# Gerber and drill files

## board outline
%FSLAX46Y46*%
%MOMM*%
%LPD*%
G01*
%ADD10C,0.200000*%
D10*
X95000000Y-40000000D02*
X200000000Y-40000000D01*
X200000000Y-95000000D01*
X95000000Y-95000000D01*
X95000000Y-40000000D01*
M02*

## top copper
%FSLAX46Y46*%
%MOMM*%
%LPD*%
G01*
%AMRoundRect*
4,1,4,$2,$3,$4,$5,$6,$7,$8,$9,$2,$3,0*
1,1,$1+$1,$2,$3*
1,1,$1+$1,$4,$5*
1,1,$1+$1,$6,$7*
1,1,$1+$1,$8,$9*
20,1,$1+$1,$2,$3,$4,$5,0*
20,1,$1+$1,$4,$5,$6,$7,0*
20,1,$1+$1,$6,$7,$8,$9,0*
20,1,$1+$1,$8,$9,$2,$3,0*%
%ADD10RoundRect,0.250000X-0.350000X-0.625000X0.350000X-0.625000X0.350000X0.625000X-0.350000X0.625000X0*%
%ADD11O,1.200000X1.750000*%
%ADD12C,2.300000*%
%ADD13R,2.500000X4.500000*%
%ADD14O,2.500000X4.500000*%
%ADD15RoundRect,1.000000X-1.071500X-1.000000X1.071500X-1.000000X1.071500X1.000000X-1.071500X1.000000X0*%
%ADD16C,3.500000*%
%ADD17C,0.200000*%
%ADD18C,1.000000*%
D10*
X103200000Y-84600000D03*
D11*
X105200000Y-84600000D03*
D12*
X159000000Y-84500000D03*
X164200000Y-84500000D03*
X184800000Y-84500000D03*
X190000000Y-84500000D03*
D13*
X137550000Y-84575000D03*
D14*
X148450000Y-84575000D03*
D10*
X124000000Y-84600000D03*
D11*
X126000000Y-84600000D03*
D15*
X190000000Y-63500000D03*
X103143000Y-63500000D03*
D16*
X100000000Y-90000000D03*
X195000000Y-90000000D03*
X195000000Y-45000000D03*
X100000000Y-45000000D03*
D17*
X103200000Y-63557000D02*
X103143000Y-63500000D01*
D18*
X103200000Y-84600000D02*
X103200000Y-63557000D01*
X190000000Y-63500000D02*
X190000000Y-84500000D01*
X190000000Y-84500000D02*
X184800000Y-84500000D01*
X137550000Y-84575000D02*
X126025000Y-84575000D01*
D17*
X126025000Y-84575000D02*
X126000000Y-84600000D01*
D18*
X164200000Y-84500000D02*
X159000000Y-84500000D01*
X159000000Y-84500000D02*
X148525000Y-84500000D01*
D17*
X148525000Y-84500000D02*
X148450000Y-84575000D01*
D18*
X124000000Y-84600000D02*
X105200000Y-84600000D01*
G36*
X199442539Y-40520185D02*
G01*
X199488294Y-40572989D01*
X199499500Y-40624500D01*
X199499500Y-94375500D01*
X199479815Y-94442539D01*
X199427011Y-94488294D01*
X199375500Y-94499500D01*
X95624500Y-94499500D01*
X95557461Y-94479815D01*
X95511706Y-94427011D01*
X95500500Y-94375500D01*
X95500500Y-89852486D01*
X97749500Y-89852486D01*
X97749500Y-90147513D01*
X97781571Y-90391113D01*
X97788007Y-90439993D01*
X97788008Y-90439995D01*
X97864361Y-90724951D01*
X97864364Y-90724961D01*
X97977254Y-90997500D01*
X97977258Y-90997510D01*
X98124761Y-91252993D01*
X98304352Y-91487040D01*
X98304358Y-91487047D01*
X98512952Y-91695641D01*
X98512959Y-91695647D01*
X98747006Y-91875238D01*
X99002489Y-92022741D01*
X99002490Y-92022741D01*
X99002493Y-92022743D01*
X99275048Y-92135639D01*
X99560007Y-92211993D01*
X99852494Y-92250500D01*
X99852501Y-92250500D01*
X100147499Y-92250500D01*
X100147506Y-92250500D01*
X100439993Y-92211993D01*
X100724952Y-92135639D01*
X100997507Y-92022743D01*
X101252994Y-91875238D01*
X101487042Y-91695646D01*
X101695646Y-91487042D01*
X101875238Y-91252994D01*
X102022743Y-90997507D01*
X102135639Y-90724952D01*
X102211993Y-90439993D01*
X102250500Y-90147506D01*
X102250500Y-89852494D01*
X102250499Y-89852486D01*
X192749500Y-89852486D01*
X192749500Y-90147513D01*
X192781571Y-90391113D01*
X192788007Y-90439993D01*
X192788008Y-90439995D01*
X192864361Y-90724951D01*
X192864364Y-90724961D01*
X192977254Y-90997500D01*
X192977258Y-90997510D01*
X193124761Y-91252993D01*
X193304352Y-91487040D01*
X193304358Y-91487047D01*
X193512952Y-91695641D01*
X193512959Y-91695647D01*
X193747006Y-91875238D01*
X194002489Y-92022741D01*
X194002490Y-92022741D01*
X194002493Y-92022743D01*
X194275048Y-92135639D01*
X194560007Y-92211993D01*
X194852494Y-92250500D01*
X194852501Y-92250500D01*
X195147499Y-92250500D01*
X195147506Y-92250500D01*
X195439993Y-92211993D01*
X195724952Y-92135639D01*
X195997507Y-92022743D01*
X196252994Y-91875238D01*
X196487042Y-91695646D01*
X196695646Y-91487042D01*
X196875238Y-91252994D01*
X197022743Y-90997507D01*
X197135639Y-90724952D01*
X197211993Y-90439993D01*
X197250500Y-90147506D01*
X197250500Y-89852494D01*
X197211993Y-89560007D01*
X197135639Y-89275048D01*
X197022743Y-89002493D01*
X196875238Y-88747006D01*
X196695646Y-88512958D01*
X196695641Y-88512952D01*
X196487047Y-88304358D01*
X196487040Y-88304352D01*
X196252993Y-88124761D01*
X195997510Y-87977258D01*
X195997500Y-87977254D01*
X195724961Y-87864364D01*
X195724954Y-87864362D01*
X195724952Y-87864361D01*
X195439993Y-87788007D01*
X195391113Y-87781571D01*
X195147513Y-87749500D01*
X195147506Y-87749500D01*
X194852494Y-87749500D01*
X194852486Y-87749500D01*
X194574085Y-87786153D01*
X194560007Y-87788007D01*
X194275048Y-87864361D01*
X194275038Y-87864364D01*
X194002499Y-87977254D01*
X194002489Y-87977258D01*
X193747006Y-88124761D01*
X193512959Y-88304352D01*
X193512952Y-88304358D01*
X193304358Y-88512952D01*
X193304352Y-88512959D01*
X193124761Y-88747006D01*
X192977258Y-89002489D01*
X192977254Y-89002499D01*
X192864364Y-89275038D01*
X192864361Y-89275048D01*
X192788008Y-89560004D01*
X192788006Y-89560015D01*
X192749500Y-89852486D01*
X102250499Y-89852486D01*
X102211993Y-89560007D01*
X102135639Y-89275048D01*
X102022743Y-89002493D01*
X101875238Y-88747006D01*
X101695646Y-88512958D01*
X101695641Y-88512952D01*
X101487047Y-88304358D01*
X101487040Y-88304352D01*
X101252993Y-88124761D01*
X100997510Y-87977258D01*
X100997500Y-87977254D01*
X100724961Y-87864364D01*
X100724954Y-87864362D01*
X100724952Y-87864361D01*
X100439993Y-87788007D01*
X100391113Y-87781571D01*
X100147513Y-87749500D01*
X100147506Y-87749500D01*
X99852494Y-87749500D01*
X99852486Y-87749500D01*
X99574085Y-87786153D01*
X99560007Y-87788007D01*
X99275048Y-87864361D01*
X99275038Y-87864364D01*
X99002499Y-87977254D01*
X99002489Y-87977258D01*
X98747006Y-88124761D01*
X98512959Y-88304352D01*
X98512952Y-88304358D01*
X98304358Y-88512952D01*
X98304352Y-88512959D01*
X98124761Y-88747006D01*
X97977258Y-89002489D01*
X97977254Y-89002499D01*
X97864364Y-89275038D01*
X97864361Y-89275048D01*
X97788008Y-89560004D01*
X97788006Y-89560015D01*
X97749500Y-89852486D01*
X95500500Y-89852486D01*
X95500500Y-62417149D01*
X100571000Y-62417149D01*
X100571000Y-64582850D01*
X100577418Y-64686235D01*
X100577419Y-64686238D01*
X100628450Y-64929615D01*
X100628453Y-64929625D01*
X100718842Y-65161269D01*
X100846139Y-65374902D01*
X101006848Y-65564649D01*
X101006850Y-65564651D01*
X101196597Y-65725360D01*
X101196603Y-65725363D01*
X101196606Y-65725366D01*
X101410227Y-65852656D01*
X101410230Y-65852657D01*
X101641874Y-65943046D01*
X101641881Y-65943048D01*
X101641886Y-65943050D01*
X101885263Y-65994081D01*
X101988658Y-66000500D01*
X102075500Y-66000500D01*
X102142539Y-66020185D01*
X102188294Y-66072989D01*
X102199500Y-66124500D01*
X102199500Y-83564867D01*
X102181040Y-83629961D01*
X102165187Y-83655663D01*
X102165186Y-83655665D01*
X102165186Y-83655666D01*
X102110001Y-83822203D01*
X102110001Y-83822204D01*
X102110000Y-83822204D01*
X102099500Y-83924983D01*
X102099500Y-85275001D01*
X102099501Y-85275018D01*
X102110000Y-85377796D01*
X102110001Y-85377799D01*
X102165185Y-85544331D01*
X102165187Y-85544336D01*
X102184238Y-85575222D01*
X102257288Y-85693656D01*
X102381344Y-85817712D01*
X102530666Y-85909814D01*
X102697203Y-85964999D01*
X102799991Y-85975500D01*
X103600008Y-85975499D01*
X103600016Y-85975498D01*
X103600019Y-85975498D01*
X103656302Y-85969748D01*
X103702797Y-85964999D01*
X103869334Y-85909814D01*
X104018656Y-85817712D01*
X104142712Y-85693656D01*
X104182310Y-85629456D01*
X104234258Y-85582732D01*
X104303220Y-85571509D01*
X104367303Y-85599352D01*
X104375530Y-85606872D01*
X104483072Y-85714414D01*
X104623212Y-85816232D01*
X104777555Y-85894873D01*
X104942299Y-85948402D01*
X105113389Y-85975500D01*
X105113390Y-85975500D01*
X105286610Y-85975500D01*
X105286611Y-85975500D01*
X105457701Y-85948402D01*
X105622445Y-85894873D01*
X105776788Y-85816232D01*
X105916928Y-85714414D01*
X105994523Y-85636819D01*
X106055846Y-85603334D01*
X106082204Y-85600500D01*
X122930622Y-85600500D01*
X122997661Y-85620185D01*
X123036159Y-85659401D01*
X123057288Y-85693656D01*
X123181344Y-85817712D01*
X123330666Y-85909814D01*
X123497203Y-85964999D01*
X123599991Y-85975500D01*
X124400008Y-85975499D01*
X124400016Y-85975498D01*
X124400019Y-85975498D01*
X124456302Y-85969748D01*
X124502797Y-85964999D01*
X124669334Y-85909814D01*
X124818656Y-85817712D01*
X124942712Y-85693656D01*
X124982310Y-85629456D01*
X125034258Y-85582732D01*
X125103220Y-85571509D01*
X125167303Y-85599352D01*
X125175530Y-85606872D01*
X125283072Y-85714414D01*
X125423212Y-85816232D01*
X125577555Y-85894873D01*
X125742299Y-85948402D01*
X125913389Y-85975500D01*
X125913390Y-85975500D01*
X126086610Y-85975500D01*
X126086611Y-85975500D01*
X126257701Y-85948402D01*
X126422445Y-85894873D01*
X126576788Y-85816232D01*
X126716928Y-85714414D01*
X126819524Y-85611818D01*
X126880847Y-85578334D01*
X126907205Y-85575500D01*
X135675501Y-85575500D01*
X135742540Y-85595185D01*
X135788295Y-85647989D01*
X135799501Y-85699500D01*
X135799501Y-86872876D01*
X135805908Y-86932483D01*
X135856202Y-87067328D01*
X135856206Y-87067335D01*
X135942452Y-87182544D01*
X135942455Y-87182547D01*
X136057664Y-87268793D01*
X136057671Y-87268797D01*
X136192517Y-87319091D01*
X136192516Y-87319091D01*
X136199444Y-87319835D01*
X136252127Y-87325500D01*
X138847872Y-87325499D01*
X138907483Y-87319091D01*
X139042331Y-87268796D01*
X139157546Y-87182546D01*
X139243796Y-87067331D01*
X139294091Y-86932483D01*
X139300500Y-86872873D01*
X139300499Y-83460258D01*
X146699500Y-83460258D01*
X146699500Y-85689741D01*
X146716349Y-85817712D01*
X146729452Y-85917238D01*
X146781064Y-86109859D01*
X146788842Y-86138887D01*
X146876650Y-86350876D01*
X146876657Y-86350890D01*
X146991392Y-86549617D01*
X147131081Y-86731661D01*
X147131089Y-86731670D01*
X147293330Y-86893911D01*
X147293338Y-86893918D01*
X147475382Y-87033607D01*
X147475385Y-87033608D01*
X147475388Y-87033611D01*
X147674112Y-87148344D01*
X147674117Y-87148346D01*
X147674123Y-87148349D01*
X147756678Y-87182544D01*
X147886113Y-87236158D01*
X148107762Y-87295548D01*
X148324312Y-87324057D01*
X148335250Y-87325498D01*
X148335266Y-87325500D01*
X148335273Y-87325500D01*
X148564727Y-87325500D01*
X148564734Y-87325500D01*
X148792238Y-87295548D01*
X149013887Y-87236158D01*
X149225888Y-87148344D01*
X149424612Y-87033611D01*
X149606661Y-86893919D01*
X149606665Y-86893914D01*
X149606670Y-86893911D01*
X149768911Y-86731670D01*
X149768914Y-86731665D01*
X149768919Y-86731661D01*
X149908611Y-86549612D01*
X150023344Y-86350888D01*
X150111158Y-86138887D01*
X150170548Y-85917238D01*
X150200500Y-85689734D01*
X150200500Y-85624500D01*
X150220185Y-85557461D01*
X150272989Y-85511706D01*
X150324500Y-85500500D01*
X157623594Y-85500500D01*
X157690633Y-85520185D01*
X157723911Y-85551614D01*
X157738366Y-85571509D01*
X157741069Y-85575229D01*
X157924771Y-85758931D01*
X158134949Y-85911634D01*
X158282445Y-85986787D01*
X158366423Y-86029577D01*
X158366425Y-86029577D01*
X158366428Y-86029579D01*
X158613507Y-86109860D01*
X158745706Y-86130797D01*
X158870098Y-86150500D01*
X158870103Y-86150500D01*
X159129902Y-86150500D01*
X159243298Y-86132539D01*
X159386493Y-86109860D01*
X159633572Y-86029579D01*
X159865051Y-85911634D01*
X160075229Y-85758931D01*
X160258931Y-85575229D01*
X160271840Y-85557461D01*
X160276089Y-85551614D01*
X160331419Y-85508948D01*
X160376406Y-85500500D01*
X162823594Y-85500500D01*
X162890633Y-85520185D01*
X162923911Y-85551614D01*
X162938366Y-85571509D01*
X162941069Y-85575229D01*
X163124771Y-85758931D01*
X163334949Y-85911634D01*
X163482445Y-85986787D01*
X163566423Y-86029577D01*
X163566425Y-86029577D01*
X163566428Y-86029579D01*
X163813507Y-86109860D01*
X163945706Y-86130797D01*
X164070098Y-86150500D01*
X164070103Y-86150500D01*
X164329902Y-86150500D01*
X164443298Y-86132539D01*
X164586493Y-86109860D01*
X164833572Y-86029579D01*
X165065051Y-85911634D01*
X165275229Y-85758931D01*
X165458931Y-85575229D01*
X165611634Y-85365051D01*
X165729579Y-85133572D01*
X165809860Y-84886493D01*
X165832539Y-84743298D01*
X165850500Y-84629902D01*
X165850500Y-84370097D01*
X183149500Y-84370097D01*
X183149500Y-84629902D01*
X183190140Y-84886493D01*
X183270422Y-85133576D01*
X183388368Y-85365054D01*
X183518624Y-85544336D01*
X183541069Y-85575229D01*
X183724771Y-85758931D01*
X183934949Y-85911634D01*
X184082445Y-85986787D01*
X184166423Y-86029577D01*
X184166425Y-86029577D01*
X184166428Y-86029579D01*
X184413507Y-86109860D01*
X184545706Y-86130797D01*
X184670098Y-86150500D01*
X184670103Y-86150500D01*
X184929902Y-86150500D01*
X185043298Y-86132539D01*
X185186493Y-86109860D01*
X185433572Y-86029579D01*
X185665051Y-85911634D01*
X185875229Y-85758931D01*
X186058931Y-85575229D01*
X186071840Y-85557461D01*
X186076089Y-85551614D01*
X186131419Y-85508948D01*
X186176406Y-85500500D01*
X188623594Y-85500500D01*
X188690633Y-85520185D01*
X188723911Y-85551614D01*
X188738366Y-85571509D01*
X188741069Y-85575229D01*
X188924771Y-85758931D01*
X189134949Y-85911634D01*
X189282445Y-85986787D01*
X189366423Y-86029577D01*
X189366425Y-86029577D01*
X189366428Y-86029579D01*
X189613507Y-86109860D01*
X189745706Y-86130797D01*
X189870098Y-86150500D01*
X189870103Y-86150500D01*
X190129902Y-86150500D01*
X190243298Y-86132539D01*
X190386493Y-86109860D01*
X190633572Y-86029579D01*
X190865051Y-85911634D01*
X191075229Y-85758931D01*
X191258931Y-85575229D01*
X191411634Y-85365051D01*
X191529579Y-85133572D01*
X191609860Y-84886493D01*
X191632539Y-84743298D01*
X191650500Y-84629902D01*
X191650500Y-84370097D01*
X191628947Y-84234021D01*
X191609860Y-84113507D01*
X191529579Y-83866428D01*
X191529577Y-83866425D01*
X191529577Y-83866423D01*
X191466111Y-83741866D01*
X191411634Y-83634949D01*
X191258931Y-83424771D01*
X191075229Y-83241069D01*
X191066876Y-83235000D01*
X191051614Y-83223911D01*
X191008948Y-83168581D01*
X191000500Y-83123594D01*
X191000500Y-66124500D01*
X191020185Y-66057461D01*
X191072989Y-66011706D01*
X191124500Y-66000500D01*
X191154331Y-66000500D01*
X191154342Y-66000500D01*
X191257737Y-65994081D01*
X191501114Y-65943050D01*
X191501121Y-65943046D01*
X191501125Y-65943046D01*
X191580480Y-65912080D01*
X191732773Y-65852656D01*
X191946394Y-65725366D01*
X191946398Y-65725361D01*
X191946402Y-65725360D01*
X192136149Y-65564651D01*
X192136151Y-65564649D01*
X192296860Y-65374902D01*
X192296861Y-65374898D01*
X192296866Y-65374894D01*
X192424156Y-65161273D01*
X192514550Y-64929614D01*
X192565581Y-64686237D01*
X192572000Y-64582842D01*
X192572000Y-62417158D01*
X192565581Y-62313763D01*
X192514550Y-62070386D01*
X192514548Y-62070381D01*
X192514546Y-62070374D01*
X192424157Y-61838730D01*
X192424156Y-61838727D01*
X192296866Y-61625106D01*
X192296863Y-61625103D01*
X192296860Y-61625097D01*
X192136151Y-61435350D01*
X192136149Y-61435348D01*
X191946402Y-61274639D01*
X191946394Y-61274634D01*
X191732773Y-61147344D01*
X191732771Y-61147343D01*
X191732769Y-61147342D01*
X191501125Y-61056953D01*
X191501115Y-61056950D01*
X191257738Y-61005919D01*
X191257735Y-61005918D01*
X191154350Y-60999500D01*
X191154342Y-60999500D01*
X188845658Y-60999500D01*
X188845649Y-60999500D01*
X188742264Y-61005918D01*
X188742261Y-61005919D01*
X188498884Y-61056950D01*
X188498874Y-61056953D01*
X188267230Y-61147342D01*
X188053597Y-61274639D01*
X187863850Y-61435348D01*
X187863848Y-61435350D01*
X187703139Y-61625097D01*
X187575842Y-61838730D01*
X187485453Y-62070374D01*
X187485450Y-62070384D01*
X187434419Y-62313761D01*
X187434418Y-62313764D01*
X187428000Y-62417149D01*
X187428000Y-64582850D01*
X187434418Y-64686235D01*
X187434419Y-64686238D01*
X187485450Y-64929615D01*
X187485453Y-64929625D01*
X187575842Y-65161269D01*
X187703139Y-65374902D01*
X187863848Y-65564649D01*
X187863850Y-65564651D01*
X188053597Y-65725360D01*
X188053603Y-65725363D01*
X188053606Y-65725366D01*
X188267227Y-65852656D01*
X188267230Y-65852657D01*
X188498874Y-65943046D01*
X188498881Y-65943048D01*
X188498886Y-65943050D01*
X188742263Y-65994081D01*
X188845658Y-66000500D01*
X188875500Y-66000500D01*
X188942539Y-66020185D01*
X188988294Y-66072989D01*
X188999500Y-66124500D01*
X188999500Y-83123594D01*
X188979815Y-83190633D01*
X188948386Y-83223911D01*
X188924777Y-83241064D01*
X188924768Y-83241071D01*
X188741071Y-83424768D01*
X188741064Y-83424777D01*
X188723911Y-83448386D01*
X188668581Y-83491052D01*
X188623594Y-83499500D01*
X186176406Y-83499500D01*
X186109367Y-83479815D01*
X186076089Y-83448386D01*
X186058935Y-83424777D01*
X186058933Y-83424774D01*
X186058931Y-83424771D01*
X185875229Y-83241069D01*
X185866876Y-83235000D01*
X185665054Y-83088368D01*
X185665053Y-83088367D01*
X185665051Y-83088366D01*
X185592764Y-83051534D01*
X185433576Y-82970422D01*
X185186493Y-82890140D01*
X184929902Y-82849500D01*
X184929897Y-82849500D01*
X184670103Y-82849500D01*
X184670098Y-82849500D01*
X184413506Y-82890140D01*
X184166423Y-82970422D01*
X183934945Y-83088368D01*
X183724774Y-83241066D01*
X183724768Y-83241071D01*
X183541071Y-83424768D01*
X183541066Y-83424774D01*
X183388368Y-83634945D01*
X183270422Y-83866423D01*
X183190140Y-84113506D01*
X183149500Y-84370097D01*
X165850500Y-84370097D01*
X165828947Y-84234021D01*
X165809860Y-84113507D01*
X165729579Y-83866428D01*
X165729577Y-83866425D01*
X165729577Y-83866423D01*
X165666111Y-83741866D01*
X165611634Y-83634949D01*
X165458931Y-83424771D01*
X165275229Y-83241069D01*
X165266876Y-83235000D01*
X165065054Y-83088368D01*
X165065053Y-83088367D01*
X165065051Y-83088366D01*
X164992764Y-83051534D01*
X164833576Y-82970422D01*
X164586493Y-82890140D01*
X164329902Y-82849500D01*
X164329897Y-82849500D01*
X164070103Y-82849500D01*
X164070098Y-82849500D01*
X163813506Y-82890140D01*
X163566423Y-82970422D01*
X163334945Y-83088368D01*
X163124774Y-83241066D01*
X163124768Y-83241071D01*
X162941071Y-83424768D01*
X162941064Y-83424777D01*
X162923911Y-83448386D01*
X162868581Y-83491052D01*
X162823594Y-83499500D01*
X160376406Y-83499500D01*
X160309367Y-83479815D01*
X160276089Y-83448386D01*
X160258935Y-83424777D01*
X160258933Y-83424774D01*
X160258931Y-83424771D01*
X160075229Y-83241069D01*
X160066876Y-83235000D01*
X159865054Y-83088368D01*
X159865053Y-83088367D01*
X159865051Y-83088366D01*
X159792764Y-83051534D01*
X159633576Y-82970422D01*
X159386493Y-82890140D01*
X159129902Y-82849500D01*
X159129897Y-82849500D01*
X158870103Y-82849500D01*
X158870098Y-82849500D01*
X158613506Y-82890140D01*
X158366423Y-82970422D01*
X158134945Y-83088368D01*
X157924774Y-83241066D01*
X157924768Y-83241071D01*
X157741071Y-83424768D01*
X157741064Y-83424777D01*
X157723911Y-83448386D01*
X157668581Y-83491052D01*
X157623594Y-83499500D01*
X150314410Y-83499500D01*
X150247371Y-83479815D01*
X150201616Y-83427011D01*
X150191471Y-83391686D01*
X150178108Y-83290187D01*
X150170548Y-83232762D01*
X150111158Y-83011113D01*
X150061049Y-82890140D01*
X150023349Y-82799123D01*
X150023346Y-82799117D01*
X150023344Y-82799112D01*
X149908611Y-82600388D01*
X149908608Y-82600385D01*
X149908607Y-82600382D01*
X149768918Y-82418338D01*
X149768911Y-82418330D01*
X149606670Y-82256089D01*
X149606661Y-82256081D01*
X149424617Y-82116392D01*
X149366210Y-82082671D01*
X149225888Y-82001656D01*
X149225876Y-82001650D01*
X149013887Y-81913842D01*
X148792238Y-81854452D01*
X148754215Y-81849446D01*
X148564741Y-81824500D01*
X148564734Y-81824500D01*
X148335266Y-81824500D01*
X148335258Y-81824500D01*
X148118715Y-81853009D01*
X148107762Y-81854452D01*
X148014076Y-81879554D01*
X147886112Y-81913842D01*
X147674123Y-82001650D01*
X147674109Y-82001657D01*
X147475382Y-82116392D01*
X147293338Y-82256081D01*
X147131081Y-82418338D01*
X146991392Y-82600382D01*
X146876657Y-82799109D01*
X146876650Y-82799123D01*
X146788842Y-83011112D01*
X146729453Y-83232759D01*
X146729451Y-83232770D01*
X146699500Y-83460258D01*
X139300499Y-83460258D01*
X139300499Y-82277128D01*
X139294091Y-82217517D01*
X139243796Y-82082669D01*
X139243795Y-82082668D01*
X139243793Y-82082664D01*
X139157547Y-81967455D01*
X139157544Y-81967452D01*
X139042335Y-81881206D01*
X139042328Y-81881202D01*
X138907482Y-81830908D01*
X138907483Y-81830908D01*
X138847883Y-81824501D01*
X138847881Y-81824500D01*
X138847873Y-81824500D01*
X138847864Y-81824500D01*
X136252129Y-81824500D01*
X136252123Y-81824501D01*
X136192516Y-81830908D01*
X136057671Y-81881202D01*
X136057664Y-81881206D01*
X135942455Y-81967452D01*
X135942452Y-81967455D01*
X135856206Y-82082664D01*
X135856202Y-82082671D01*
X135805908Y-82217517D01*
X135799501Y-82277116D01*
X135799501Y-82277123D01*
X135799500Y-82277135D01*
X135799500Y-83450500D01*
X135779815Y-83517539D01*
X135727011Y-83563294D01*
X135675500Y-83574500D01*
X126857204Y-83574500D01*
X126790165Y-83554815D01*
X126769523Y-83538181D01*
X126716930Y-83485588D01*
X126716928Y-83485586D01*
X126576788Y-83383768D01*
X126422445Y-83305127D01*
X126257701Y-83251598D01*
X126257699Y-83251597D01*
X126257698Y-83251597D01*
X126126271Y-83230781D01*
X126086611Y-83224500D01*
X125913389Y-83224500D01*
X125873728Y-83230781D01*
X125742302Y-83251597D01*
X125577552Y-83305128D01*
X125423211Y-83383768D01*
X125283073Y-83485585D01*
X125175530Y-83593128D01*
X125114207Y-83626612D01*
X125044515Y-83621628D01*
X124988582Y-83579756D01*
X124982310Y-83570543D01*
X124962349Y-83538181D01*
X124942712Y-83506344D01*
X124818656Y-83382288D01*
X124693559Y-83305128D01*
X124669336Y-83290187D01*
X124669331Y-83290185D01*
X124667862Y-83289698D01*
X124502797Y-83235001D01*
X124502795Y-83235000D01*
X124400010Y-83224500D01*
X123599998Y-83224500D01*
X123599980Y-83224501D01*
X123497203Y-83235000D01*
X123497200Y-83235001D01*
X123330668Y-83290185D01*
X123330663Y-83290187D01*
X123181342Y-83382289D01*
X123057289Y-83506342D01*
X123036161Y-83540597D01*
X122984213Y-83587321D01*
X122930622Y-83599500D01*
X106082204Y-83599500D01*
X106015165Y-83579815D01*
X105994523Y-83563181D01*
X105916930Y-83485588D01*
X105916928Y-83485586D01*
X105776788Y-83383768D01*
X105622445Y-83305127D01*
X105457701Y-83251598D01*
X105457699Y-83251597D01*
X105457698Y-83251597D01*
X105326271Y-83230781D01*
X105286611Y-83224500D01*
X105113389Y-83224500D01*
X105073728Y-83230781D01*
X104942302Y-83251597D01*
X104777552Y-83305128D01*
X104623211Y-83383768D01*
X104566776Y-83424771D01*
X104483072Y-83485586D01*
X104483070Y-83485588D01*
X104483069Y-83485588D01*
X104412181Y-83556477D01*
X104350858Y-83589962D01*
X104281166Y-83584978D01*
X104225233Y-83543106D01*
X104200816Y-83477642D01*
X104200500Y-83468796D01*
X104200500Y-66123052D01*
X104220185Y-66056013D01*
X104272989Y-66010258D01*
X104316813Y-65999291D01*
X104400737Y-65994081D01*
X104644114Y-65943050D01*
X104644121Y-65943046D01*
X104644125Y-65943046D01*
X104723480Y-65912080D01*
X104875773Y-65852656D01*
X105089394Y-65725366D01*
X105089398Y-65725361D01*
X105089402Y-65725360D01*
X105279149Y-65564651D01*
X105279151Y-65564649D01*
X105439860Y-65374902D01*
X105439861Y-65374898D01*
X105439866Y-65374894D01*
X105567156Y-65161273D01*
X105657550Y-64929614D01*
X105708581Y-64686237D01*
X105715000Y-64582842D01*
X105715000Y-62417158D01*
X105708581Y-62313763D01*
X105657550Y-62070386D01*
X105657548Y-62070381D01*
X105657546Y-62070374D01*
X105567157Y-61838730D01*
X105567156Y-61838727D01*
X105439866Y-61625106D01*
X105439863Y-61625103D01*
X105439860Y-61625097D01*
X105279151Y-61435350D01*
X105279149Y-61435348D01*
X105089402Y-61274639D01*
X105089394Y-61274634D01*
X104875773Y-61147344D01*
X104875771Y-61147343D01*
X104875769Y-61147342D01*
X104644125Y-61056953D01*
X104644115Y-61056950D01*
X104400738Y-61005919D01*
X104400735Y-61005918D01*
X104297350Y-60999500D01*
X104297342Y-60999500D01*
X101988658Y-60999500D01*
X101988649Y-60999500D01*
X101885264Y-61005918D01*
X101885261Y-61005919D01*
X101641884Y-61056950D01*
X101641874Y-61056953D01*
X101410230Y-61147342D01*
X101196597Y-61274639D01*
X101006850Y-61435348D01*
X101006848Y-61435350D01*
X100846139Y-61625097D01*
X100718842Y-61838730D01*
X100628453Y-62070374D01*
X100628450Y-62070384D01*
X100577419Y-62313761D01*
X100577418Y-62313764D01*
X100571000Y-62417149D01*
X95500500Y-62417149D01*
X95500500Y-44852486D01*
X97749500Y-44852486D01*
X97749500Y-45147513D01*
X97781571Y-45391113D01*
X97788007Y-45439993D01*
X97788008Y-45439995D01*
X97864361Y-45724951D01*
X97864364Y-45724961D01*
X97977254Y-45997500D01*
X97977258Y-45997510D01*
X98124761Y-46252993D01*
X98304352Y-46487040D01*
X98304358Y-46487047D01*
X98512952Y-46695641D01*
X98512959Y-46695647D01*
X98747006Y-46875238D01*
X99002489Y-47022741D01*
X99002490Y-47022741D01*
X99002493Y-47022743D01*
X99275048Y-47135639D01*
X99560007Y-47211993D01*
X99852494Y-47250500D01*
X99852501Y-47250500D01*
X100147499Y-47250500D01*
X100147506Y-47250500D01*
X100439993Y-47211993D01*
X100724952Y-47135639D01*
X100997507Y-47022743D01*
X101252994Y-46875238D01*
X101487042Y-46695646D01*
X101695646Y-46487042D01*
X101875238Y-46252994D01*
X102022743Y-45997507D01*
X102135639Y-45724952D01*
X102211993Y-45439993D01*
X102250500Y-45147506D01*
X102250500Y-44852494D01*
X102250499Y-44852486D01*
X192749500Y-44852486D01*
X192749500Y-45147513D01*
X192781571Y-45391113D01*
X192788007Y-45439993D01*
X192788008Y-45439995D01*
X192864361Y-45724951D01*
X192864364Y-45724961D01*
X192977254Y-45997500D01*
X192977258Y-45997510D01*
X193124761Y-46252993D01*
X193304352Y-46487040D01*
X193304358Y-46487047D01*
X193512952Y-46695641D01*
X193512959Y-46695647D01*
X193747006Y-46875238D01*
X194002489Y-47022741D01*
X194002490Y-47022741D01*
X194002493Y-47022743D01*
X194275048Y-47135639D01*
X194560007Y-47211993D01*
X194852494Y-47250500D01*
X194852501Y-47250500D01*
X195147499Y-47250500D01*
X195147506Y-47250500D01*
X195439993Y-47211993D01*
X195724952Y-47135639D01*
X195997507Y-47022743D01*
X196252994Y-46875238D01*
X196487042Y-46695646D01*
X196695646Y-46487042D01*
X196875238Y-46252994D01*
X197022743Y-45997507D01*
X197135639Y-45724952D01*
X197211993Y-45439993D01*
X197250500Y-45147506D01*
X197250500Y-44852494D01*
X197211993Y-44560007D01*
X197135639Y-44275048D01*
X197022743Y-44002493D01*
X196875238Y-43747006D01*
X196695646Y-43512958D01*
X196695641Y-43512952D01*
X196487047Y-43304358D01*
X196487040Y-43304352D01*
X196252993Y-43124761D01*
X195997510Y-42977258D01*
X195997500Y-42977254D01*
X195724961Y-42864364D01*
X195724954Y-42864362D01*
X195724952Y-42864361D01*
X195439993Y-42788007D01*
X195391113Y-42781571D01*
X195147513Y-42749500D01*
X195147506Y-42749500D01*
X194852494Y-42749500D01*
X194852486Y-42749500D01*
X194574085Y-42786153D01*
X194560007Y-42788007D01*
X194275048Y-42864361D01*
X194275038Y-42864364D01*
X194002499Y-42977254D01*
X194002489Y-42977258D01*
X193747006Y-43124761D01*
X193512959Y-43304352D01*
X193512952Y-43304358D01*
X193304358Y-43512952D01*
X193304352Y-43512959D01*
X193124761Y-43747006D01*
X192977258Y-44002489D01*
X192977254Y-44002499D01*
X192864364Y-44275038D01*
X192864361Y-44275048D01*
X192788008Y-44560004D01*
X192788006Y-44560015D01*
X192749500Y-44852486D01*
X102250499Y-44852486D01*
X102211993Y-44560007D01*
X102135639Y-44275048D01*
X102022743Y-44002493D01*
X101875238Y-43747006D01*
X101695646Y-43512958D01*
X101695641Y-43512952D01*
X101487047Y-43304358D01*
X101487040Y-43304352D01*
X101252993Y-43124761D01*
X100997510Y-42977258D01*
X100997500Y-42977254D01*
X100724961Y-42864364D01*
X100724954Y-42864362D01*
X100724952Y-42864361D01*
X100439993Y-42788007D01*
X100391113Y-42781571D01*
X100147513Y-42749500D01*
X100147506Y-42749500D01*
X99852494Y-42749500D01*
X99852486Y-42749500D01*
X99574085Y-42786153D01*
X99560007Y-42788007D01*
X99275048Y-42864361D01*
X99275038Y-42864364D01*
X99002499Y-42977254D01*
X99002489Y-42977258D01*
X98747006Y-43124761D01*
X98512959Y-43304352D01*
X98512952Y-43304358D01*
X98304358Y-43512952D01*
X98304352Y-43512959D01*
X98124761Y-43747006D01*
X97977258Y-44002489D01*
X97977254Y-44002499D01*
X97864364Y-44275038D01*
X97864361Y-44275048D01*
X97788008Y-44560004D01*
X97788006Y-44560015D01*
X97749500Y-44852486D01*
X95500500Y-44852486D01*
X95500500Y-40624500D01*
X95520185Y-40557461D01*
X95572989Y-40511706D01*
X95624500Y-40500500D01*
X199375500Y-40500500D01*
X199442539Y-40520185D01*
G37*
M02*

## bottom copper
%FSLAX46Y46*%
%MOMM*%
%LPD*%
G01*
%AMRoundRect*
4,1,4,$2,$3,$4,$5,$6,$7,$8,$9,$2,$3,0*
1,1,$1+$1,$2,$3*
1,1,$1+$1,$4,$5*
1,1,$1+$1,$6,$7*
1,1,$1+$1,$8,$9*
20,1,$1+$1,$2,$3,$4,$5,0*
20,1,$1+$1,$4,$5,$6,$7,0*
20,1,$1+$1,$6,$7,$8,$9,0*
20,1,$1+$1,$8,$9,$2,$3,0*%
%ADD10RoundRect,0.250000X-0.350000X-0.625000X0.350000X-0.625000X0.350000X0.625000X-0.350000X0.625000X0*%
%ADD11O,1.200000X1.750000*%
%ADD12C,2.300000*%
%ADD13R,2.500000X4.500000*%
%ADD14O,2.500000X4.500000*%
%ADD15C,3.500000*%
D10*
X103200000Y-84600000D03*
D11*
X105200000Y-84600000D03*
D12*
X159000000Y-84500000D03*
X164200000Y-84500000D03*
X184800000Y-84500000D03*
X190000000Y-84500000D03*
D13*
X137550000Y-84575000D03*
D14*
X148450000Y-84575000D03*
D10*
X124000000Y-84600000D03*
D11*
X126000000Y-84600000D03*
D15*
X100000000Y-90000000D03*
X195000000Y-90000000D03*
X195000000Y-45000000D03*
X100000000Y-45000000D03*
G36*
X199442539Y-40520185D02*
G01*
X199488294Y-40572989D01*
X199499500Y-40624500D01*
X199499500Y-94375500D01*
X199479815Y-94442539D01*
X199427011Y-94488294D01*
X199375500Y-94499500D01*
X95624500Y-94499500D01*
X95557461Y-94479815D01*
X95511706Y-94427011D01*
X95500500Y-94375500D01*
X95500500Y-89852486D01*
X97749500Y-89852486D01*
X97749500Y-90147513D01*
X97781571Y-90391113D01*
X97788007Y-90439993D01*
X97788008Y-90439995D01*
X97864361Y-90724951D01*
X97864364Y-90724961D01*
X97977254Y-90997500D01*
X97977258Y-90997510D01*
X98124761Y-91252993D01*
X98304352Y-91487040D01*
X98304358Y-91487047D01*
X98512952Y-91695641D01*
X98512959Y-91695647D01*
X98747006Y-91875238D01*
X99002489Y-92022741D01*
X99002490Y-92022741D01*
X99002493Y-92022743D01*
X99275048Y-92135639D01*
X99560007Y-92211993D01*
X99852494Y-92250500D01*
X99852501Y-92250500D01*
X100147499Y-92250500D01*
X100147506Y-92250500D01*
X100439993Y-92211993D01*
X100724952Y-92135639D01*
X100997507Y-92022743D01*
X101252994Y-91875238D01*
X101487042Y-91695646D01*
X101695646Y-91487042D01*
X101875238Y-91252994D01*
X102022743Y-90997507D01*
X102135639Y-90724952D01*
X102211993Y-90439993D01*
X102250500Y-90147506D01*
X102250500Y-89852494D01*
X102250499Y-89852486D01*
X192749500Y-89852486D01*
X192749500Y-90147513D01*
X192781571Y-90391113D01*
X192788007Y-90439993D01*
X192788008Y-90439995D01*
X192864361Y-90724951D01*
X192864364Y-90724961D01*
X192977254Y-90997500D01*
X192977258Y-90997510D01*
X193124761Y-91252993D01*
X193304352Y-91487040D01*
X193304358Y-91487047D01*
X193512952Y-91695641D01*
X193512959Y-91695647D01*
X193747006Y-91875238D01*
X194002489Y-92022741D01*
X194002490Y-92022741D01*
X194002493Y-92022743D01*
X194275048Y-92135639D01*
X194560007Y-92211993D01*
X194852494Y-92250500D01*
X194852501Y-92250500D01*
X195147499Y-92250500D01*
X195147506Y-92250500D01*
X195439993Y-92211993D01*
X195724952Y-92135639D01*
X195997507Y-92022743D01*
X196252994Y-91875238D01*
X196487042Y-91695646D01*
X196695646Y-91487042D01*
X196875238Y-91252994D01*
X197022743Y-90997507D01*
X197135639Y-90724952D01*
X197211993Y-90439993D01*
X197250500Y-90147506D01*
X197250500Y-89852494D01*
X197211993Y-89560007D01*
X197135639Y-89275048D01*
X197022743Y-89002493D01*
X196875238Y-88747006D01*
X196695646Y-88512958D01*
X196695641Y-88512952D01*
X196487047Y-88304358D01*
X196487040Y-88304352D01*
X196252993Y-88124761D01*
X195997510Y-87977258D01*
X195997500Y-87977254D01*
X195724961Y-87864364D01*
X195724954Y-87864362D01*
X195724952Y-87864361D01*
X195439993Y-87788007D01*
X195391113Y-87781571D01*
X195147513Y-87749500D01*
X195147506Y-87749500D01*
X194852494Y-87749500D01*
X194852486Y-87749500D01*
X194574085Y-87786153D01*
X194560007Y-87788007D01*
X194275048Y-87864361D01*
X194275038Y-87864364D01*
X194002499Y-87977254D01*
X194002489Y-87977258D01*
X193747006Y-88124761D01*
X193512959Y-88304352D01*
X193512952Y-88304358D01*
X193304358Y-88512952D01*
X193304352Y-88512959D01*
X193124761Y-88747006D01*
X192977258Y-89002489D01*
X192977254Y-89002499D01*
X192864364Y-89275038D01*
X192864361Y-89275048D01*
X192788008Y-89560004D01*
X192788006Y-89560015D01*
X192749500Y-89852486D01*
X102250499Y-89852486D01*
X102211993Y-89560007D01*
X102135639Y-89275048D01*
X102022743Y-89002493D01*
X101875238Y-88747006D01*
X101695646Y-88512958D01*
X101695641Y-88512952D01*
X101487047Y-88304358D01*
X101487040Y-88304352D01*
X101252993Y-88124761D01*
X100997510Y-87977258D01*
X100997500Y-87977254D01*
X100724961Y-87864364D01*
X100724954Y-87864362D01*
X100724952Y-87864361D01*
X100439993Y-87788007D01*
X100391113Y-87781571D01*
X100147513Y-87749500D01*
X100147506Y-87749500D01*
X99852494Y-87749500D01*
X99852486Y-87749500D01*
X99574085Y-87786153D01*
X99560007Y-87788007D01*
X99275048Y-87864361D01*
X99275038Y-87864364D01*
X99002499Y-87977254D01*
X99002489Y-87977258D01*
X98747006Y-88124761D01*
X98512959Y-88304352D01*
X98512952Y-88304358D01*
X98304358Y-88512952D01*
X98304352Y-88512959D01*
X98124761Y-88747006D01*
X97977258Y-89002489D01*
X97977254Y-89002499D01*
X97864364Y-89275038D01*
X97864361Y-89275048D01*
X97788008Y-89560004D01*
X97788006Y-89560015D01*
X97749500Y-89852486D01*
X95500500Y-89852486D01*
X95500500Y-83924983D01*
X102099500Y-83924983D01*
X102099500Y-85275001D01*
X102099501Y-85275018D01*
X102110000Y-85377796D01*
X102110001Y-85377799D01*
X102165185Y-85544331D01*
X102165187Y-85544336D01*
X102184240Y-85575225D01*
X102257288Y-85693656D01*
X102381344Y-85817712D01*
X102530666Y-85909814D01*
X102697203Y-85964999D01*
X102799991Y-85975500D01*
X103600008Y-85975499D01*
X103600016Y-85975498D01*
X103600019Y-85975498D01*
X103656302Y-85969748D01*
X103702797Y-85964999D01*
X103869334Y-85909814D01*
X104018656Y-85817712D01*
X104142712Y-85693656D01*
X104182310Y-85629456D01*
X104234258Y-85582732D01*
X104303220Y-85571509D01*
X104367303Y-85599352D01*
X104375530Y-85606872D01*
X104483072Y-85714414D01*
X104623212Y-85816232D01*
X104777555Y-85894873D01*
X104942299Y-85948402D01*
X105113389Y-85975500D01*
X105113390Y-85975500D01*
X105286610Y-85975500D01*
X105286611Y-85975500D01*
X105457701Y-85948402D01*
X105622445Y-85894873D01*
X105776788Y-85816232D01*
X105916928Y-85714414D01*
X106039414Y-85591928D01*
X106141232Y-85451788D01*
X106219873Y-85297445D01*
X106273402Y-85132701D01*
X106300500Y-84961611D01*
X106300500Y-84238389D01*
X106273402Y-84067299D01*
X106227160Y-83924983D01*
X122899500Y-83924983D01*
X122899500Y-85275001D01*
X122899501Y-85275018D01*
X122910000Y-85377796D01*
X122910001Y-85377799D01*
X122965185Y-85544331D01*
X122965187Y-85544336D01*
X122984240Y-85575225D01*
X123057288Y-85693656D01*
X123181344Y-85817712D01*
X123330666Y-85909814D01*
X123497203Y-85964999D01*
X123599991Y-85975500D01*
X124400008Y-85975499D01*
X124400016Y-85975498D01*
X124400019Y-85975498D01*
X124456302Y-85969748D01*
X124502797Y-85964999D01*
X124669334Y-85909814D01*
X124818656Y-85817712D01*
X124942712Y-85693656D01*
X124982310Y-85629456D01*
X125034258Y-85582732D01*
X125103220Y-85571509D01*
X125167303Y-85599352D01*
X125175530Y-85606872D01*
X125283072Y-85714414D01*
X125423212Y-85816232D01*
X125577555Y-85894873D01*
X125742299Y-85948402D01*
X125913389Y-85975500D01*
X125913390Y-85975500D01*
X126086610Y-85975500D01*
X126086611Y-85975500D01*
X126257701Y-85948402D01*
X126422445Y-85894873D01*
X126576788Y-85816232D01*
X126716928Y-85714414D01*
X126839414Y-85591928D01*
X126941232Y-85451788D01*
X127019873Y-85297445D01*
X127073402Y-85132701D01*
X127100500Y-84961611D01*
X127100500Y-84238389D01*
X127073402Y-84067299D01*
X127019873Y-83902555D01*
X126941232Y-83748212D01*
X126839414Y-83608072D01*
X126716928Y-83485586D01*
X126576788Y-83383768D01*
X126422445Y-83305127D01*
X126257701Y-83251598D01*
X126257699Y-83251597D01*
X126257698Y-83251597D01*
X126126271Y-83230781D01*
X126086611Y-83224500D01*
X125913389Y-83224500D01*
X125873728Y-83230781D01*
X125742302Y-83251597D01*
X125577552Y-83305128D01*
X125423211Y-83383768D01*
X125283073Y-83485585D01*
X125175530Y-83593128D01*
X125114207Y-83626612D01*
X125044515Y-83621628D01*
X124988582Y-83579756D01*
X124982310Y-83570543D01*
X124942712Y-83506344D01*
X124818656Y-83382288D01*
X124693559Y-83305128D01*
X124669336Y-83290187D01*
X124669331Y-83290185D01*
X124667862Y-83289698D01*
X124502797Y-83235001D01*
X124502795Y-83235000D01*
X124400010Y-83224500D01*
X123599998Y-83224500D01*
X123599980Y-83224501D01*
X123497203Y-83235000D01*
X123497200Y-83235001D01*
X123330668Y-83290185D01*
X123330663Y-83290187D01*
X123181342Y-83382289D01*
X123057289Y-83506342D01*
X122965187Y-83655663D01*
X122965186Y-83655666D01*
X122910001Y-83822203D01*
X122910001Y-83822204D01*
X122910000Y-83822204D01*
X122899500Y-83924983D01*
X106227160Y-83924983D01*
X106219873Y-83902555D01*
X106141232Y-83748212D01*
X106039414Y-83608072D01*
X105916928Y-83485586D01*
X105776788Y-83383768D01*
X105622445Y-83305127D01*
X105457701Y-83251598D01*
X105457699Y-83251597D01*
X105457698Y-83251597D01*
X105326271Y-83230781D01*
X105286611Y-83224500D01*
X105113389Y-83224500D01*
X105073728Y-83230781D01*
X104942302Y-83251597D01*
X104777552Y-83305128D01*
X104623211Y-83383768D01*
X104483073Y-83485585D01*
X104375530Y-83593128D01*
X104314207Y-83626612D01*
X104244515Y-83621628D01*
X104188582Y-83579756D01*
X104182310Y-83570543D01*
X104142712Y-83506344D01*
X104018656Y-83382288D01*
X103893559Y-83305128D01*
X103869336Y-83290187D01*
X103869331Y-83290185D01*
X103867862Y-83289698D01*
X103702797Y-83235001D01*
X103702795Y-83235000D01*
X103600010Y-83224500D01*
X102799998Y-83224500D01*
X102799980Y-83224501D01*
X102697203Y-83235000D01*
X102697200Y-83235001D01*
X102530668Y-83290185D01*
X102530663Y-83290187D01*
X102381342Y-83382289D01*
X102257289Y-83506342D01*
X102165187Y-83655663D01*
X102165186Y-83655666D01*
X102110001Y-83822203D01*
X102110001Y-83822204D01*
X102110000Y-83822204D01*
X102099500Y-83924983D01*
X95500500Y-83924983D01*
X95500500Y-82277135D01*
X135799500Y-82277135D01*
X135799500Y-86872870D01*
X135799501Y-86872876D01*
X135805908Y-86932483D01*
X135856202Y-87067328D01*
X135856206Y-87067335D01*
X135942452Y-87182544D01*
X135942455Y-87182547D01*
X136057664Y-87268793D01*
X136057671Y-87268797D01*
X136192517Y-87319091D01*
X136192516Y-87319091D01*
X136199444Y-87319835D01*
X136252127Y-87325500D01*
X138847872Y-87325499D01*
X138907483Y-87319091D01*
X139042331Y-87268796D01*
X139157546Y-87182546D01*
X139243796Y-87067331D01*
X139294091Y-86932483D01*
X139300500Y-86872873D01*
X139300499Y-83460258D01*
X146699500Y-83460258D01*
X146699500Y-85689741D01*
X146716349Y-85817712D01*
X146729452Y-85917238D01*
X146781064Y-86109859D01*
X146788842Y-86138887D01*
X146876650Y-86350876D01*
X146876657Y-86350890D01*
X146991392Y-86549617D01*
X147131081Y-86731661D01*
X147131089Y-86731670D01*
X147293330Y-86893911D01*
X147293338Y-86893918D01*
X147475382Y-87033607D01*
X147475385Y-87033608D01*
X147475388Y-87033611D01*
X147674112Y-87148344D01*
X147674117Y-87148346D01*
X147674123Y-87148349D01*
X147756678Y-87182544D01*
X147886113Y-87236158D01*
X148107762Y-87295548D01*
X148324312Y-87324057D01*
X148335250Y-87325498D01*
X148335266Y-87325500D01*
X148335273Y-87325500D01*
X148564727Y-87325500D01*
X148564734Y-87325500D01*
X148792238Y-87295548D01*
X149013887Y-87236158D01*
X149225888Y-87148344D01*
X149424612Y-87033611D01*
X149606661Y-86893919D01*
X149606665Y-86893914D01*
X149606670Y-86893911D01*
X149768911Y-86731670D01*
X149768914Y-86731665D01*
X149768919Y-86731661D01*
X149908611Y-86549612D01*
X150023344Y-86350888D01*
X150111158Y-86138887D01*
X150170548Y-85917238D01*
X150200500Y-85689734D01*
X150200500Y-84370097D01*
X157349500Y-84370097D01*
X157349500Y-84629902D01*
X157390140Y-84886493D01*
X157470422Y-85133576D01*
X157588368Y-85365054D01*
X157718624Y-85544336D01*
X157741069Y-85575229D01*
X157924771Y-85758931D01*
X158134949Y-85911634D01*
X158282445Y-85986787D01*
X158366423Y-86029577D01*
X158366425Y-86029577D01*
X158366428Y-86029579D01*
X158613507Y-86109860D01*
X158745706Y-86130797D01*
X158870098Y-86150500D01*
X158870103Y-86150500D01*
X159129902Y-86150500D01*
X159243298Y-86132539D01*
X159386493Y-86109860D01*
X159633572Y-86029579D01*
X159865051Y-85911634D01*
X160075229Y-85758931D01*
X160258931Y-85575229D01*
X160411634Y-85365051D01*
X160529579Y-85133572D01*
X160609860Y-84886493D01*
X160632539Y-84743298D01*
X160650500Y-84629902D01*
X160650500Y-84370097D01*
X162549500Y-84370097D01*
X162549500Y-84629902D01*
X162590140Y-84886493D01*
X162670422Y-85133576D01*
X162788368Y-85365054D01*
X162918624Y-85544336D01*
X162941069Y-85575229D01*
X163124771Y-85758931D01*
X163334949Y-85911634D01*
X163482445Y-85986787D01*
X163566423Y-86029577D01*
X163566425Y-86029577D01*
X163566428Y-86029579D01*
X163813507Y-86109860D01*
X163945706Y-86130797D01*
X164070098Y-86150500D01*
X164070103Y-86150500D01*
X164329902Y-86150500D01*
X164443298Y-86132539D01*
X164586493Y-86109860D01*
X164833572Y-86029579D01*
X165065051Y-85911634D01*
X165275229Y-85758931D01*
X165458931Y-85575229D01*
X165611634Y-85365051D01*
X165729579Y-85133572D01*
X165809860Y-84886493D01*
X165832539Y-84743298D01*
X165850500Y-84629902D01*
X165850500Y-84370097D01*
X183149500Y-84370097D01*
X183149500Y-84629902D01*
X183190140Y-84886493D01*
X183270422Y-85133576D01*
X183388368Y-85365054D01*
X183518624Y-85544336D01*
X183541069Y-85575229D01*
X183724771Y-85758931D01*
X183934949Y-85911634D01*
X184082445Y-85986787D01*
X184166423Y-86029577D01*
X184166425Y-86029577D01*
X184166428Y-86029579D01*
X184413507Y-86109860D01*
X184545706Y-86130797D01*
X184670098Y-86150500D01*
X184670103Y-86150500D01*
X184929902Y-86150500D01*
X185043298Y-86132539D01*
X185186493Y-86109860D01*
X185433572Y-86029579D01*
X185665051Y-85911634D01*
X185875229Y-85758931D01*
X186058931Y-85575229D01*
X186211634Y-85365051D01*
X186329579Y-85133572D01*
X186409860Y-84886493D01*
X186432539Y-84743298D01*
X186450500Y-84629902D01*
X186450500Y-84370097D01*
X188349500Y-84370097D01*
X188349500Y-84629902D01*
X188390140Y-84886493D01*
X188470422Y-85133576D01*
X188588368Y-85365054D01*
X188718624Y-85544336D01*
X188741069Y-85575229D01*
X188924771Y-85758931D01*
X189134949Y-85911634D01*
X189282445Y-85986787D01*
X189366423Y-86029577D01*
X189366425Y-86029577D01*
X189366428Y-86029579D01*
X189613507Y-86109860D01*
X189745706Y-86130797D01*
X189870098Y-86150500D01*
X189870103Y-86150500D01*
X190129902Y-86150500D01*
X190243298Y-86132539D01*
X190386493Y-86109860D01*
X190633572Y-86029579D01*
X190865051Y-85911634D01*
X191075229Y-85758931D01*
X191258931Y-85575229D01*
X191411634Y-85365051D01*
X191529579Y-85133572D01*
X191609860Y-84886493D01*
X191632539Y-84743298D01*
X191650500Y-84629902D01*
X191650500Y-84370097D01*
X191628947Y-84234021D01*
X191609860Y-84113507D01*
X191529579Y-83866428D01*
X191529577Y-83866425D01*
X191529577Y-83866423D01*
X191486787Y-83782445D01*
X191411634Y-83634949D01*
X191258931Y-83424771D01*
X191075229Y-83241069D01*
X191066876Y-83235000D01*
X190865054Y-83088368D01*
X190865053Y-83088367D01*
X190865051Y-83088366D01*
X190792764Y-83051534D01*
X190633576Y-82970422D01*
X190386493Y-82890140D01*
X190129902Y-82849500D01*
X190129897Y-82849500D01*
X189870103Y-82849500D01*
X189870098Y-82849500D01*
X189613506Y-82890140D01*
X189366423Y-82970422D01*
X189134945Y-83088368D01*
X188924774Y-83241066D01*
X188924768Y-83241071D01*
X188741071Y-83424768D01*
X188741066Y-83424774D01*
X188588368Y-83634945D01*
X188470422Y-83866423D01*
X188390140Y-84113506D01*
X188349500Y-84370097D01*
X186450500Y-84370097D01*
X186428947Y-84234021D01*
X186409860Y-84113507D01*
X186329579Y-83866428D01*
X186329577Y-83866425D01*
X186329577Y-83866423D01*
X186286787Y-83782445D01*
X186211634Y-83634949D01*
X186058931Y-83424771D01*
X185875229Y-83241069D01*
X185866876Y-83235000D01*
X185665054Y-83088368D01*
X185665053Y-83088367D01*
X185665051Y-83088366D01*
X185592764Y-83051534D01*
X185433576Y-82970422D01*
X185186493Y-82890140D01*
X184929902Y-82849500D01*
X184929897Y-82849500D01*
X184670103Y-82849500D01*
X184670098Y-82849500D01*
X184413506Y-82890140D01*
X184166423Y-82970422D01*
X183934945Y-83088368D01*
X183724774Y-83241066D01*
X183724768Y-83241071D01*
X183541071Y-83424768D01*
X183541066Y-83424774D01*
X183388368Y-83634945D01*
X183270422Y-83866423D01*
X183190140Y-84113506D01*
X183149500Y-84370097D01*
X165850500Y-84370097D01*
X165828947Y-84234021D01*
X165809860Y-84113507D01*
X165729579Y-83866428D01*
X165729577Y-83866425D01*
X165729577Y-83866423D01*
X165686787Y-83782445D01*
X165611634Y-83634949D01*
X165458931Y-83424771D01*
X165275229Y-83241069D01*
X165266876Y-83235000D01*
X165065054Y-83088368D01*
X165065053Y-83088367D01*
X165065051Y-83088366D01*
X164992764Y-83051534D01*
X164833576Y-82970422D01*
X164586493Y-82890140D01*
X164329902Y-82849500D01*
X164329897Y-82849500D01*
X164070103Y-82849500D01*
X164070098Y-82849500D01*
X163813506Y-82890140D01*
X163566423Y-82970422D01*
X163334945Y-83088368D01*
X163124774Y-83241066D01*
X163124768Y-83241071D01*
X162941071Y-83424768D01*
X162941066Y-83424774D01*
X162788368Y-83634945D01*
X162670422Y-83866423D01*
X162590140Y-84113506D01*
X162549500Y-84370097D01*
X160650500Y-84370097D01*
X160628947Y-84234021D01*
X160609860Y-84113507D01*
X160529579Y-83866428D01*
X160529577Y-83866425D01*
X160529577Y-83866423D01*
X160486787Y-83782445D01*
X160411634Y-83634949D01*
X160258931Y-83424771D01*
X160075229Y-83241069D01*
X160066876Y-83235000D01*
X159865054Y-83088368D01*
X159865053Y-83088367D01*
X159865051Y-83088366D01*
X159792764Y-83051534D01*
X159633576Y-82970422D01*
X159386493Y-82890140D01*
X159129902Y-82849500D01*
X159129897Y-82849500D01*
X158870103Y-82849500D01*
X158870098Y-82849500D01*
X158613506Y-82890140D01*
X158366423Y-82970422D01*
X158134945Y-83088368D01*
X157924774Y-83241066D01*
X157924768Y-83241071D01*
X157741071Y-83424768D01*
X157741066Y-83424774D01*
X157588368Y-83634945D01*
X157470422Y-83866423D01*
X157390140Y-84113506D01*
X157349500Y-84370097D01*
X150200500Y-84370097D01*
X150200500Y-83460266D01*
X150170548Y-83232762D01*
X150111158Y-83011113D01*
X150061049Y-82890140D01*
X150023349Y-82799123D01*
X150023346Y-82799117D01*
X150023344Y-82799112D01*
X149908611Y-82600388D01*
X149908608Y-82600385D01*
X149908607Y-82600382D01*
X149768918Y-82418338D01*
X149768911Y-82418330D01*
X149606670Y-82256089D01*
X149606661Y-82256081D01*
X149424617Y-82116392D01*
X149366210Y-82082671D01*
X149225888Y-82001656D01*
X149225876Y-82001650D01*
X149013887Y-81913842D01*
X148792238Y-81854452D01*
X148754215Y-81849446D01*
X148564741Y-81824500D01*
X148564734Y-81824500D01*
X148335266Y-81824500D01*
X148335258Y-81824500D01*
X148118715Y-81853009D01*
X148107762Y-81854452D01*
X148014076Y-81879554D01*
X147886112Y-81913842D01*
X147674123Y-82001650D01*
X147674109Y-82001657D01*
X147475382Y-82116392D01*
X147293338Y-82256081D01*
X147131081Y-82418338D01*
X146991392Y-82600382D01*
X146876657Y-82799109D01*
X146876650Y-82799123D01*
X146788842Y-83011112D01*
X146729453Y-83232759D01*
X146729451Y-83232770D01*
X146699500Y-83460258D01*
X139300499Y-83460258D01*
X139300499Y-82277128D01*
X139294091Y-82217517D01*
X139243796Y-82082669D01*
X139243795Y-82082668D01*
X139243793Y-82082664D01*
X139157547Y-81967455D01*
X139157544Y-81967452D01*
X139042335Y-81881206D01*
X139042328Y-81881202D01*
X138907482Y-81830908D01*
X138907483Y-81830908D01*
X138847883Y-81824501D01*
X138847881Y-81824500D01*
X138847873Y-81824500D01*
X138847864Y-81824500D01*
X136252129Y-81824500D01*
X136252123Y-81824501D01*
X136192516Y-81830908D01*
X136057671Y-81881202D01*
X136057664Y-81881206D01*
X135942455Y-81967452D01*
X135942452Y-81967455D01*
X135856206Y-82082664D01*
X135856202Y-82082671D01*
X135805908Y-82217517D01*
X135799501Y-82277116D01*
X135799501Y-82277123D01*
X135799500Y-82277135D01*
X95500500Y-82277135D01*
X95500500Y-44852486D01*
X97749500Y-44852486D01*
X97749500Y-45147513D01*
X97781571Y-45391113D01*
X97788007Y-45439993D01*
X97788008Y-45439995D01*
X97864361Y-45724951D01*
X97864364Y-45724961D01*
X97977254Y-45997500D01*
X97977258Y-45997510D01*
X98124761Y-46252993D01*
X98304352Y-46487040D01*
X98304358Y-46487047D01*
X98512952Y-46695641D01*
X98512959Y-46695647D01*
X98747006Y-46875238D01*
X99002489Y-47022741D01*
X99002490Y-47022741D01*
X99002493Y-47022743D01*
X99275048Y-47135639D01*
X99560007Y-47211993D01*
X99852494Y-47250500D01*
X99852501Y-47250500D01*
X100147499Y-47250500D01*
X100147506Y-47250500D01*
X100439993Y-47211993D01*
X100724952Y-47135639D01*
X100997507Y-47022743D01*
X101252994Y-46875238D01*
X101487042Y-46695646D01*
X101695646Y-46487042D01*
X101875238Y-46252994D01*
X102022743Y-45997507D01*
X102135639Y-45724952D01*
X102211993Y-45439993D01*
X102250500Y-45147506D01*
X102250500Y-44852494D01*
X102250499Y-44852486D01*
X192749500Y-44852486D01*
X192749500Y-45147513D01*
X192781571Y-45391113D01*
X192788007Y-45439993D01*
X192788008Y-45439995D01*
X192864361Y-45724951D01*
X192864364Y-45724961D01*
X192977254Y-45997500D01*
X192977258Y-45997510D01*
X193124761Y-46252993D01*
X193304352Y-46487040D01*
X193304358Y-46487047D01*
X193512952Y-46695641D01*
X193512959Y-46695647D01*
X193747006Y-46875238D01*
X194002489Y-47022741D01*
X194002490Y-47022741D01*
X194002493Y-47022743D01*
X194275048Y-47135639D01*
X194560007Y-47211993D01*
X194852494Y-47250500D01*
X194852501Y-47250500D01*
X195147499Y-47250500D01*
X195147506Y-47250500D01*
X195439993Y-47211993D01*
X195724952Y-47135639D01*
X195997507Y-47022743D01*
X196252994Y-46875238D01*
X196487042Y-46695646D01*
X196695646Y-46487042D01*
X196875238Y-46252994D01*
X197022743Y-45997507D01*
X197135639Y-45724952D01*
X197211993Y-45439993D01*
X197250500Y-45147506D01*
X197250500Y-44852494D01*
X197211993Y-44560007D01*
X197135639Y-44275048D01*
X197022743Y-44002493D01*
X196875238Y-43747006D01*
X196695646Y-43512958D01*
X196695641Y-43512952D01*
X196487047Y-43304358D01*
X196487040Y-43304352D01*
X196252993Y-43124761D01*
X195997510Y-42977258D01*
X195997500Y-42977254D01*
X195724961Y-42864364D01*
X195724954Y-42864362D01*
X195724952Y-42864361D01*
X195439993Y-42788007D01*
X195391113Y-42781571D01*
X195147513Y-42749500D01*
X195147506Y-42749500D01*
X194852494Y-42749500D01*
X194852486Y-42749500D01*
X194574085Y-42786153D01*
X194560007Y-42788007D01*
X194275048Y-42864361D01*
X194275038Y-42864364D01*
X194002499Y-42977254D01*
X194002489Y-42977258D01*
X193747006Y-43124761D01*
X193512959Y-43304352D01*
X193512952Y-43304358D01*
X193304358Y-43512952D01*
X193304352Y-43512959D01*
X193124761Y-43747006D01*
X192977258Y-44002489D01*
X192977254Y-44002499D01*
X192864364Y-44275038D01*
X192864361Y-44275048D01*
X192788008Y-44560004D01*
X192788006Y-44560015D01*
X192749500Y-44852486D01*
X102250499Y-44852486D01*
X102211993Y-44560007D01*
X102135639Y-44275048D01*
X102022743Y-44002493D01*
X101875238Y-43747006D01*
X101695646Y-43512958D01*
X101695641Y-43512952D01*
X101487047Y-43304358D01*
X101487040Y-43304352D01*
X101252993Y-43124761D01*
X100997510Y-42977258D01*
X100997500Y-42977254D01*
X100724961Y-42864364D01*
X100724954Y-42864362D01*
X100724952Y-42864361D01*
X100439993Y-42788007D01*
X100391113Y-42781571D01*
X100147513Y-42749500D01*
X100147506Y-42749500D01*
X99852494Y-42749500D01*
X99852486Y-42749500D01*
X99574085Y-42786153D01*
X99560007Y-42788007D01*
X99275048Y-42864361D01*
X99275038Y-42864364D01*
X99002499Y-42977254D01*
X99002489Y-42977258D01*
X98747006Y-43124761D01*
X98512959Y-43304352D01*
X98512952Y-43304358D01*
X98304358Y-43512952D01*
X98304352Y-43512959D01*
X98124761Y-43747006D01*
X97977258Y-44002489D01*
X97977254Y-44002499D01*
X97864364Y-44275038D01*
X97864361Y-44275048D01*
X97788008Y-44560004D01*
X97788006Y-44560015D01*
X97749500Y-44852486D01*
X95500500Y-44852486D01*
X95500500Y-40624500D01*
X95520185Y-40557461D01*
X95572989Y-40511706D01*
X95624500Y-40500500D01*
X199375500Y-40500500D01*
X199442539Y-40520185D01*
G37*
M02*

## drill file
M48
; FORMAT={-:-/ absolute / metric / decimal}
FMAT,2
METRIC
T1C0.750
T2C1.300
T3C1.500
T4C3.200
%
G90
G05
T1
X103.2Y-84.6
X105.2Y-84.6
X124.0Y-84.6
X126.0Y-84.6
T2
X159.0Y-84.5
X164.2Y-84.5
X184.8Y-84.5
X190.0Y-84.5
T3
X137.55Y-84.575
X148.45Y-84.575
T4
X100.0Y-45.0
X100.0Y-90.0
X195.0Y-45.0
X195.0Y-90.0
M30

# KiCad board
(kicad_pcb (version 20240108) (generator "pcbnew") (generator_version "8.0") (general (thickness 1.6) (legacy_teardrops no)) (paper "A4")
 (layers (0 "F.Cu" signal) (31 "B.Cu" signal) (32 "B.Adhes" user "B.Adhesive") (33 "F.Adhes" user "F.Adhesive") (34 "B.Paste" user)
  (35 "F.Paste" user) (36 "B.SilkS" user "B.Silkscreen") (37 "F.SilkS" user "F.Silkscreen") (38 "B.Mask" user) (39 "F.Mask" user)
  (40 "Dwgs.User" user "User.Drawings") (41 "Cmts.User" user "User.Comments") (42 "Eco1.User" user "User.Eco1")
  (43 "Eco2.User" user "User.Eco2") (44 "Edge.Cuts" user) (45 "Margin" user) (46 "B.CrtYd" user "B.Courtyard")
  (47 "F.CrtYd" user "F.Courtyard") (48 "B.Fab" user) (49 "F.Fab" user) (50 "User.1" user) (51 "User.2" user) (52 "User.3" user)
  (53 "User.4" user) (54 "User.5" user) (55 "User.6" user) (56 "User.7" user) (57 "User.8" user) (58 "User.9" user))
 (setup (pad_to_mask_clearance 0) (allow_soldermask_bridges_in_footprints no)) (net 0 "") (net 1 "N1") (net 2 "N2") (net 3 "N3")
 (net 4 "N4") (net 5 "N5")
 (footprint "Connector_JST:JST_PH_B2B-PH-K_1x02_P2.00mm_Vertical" (layer "F.Cu") (at 103.2 84.6)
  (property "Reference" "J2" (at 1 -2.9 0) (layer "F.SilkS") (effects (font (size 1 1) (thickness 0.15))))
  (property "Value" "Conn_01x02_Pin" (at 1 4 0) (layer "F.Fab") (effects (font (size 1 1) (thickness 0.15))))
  (pad "1" thru_hole roundrect (at 0 0) (size 1.2 1.75) (drill 0.75) (layers "*.Cu" "*.Mask") (remove_unused_layers no)
   (roundrect_rratio 0.208333) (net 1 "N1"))
  (pad "2" thru_hole oval (at 2 0) (size 1.2 1.75) (drill 0.75) (layers "*.Cu" "*.Mask") (remove_unused_layers no) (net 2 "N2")))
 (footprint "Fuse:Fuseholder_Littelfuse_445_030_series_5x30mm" (layer "F.Cu") (at 159 84.5)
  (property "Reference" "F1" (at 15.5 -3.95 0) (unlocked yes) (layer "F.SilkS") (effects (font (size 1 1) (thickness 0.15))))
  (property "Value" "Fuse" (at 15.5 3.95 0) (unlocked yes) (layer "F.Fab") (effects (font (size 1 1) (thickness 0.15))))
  (pad "1" thru_hole circle (at 0 0) (size 2.3 2.3) (drill 1.3) (layers "*.Cu" "*.Mask") (remove_unused_layers no) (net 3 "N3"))
  (pad "1" thru_hole circle (at 5.2 0) (size 2.3 2.3) (drill 1.3) (layers "*.Cu" "*.Mask") (remove_unused_layers no) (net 3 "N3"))
  (pad "2" thru_hole circle (at 25.8 0) (size 2.3 2.3) (drill 1.3) (layers "*.Cu" "*.Mask") (remove_unused_layers no) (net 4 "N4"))
  (pad "2" thru_hole circle (at 31 0) (size 2.3 2.3) (drill 1.3) (layers "*.Cu" "*.Mask") (remove_unused_layers no) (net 4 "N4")))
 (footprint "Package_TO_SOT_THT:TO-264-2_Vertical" (layer "F.Cu") (at 137.55 84.575)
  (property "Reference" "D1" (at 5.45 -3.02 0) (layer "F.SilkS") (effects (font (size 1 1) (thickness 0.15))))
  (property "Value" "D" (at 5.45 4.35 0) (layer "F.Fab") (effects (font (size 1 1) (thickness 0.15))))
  (pad "1" thru_hole rect (at 0 0) (size 2.5 4.5) (drill 1.5) (layers "*.Cu" "*.Mask") (remove_unused_layers no) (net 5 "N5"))
  (pad "2" thru_hole oval (at 10.9 0) (size 2.5 4.5) (drill 1.5) (layers "*.Cu" "*.Mask") (remove_unused_layers no) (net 3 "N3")))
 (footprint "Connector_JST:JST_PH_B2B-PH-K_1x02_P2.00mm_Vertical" (layer "F.Cu") (at 124 84.6)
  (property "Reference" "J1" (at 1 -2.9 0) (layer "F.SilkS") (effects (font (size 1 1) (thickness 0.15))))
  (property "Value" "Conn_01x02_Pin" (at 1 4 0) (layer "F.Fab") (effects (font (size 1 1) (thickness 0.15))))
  (pad "1" thru_hole roundrect (at 0 0) (size 1.2 1.75) (drill 0.75) (layers "*.Cu" "*.Mask") (remove_unused_layers no)
   (roundrect_rratio 0.208333) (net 2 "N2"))
  (pad "2" thru_hole oval (at 2 0) (size 1.2 1.75) (drill 0.75) (layers "*.Cu" "*.Mask") (remove_unused_layers no) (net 5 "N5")))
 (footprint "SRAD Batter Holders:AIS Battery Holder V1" (layer "F.Cu") (at 146.5715 63.5)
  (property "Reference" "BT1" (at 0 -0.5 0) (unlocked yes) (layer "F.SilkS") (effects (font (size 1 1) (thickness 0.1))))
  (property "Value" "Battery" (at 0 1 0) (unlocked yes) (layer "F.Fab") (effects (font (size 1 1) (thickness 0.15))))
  (pad "1" smd roundrect (at 43.4285 0) (size 4.143 4) (layers "F.Cu" "F.Paste" "F.Mask") (roundrect_rratio 0.25) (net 4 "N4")
   (thermal_bridge_angle 45))
  (pad "2" smd roundrect (at -43.4285 0) (size 4.143 4) (layers "F.Cu" "F.Paste" "F.Mask") (roundrect_rratio 0.25) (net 1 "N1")
   (thermal_bridge_angle 45)))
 (gr_rect (start 95 40) (end 200 95) (stroke (width 0.2) (type default)) (fill none) (layer "Edge.Cuts"))
 (via (at 100 90) (size 3.5) (drill 3.2) (layers "F.Cu" "B.Cu") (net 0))
 (via (at 195 90) (size 3.5) (drill 3.2) (layers "F.Cu" "B.Cu") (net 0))
 (via (at 195 45) (size 3.5) (drill 3.2) (layers "F.Cu" "B.Cu") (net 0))
 (via (at 100 45) (size 3.5) (drill 3.2) (layers "F.Cu" "B.Cu") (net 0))
 (segment (start 103.2 63.557) (end 103.143 63.5) (width 0.2) (layer "F.Cu") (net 1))
 (segment (start 103.2 84.6) (end 103.2 63.557) (width 1) (layer "F.Cu") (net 1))
 (segment (start 190 63.5) (end 190 84.5) (width 1) (layer "F.Cu") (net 4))
 (segment (start 190 84.5) (end 184.8 84.5) (width 1) (layer "F.Cu") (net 4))
 (segment (start 137.55 84.575) (end 126.025 84.575) (width 1) (layer "F.Cu") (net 5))
 (segment (start 126.025 84.575) (end 126 84.6) (width 0.2) (layer "F.Cu") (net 5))
 (segment (start 164.2 84.5) (end 159 84.5) (width 1) (layer "F.Cu") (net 3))
 (segment (start 159 84.5) (end 148.525 84.5) (width 1) (layer "F.Cu") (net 3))
 (segment (start 148.525 84.5) (end 148.45 84.575) (width 0.2) (layer "F.Cu") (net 3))
 (segment (start 124 84.6) (end 105.2 84.6) (width 1) (layer "F.Cu") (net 2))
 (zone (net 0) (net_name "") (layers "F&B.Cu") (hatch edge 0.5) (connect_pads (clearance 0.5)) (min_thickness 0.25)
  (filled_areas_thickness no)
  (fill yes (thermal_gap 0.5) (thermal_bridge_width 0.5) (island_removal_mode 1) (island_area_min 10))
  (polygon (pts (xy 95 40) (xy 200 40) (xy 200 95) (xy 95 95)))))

